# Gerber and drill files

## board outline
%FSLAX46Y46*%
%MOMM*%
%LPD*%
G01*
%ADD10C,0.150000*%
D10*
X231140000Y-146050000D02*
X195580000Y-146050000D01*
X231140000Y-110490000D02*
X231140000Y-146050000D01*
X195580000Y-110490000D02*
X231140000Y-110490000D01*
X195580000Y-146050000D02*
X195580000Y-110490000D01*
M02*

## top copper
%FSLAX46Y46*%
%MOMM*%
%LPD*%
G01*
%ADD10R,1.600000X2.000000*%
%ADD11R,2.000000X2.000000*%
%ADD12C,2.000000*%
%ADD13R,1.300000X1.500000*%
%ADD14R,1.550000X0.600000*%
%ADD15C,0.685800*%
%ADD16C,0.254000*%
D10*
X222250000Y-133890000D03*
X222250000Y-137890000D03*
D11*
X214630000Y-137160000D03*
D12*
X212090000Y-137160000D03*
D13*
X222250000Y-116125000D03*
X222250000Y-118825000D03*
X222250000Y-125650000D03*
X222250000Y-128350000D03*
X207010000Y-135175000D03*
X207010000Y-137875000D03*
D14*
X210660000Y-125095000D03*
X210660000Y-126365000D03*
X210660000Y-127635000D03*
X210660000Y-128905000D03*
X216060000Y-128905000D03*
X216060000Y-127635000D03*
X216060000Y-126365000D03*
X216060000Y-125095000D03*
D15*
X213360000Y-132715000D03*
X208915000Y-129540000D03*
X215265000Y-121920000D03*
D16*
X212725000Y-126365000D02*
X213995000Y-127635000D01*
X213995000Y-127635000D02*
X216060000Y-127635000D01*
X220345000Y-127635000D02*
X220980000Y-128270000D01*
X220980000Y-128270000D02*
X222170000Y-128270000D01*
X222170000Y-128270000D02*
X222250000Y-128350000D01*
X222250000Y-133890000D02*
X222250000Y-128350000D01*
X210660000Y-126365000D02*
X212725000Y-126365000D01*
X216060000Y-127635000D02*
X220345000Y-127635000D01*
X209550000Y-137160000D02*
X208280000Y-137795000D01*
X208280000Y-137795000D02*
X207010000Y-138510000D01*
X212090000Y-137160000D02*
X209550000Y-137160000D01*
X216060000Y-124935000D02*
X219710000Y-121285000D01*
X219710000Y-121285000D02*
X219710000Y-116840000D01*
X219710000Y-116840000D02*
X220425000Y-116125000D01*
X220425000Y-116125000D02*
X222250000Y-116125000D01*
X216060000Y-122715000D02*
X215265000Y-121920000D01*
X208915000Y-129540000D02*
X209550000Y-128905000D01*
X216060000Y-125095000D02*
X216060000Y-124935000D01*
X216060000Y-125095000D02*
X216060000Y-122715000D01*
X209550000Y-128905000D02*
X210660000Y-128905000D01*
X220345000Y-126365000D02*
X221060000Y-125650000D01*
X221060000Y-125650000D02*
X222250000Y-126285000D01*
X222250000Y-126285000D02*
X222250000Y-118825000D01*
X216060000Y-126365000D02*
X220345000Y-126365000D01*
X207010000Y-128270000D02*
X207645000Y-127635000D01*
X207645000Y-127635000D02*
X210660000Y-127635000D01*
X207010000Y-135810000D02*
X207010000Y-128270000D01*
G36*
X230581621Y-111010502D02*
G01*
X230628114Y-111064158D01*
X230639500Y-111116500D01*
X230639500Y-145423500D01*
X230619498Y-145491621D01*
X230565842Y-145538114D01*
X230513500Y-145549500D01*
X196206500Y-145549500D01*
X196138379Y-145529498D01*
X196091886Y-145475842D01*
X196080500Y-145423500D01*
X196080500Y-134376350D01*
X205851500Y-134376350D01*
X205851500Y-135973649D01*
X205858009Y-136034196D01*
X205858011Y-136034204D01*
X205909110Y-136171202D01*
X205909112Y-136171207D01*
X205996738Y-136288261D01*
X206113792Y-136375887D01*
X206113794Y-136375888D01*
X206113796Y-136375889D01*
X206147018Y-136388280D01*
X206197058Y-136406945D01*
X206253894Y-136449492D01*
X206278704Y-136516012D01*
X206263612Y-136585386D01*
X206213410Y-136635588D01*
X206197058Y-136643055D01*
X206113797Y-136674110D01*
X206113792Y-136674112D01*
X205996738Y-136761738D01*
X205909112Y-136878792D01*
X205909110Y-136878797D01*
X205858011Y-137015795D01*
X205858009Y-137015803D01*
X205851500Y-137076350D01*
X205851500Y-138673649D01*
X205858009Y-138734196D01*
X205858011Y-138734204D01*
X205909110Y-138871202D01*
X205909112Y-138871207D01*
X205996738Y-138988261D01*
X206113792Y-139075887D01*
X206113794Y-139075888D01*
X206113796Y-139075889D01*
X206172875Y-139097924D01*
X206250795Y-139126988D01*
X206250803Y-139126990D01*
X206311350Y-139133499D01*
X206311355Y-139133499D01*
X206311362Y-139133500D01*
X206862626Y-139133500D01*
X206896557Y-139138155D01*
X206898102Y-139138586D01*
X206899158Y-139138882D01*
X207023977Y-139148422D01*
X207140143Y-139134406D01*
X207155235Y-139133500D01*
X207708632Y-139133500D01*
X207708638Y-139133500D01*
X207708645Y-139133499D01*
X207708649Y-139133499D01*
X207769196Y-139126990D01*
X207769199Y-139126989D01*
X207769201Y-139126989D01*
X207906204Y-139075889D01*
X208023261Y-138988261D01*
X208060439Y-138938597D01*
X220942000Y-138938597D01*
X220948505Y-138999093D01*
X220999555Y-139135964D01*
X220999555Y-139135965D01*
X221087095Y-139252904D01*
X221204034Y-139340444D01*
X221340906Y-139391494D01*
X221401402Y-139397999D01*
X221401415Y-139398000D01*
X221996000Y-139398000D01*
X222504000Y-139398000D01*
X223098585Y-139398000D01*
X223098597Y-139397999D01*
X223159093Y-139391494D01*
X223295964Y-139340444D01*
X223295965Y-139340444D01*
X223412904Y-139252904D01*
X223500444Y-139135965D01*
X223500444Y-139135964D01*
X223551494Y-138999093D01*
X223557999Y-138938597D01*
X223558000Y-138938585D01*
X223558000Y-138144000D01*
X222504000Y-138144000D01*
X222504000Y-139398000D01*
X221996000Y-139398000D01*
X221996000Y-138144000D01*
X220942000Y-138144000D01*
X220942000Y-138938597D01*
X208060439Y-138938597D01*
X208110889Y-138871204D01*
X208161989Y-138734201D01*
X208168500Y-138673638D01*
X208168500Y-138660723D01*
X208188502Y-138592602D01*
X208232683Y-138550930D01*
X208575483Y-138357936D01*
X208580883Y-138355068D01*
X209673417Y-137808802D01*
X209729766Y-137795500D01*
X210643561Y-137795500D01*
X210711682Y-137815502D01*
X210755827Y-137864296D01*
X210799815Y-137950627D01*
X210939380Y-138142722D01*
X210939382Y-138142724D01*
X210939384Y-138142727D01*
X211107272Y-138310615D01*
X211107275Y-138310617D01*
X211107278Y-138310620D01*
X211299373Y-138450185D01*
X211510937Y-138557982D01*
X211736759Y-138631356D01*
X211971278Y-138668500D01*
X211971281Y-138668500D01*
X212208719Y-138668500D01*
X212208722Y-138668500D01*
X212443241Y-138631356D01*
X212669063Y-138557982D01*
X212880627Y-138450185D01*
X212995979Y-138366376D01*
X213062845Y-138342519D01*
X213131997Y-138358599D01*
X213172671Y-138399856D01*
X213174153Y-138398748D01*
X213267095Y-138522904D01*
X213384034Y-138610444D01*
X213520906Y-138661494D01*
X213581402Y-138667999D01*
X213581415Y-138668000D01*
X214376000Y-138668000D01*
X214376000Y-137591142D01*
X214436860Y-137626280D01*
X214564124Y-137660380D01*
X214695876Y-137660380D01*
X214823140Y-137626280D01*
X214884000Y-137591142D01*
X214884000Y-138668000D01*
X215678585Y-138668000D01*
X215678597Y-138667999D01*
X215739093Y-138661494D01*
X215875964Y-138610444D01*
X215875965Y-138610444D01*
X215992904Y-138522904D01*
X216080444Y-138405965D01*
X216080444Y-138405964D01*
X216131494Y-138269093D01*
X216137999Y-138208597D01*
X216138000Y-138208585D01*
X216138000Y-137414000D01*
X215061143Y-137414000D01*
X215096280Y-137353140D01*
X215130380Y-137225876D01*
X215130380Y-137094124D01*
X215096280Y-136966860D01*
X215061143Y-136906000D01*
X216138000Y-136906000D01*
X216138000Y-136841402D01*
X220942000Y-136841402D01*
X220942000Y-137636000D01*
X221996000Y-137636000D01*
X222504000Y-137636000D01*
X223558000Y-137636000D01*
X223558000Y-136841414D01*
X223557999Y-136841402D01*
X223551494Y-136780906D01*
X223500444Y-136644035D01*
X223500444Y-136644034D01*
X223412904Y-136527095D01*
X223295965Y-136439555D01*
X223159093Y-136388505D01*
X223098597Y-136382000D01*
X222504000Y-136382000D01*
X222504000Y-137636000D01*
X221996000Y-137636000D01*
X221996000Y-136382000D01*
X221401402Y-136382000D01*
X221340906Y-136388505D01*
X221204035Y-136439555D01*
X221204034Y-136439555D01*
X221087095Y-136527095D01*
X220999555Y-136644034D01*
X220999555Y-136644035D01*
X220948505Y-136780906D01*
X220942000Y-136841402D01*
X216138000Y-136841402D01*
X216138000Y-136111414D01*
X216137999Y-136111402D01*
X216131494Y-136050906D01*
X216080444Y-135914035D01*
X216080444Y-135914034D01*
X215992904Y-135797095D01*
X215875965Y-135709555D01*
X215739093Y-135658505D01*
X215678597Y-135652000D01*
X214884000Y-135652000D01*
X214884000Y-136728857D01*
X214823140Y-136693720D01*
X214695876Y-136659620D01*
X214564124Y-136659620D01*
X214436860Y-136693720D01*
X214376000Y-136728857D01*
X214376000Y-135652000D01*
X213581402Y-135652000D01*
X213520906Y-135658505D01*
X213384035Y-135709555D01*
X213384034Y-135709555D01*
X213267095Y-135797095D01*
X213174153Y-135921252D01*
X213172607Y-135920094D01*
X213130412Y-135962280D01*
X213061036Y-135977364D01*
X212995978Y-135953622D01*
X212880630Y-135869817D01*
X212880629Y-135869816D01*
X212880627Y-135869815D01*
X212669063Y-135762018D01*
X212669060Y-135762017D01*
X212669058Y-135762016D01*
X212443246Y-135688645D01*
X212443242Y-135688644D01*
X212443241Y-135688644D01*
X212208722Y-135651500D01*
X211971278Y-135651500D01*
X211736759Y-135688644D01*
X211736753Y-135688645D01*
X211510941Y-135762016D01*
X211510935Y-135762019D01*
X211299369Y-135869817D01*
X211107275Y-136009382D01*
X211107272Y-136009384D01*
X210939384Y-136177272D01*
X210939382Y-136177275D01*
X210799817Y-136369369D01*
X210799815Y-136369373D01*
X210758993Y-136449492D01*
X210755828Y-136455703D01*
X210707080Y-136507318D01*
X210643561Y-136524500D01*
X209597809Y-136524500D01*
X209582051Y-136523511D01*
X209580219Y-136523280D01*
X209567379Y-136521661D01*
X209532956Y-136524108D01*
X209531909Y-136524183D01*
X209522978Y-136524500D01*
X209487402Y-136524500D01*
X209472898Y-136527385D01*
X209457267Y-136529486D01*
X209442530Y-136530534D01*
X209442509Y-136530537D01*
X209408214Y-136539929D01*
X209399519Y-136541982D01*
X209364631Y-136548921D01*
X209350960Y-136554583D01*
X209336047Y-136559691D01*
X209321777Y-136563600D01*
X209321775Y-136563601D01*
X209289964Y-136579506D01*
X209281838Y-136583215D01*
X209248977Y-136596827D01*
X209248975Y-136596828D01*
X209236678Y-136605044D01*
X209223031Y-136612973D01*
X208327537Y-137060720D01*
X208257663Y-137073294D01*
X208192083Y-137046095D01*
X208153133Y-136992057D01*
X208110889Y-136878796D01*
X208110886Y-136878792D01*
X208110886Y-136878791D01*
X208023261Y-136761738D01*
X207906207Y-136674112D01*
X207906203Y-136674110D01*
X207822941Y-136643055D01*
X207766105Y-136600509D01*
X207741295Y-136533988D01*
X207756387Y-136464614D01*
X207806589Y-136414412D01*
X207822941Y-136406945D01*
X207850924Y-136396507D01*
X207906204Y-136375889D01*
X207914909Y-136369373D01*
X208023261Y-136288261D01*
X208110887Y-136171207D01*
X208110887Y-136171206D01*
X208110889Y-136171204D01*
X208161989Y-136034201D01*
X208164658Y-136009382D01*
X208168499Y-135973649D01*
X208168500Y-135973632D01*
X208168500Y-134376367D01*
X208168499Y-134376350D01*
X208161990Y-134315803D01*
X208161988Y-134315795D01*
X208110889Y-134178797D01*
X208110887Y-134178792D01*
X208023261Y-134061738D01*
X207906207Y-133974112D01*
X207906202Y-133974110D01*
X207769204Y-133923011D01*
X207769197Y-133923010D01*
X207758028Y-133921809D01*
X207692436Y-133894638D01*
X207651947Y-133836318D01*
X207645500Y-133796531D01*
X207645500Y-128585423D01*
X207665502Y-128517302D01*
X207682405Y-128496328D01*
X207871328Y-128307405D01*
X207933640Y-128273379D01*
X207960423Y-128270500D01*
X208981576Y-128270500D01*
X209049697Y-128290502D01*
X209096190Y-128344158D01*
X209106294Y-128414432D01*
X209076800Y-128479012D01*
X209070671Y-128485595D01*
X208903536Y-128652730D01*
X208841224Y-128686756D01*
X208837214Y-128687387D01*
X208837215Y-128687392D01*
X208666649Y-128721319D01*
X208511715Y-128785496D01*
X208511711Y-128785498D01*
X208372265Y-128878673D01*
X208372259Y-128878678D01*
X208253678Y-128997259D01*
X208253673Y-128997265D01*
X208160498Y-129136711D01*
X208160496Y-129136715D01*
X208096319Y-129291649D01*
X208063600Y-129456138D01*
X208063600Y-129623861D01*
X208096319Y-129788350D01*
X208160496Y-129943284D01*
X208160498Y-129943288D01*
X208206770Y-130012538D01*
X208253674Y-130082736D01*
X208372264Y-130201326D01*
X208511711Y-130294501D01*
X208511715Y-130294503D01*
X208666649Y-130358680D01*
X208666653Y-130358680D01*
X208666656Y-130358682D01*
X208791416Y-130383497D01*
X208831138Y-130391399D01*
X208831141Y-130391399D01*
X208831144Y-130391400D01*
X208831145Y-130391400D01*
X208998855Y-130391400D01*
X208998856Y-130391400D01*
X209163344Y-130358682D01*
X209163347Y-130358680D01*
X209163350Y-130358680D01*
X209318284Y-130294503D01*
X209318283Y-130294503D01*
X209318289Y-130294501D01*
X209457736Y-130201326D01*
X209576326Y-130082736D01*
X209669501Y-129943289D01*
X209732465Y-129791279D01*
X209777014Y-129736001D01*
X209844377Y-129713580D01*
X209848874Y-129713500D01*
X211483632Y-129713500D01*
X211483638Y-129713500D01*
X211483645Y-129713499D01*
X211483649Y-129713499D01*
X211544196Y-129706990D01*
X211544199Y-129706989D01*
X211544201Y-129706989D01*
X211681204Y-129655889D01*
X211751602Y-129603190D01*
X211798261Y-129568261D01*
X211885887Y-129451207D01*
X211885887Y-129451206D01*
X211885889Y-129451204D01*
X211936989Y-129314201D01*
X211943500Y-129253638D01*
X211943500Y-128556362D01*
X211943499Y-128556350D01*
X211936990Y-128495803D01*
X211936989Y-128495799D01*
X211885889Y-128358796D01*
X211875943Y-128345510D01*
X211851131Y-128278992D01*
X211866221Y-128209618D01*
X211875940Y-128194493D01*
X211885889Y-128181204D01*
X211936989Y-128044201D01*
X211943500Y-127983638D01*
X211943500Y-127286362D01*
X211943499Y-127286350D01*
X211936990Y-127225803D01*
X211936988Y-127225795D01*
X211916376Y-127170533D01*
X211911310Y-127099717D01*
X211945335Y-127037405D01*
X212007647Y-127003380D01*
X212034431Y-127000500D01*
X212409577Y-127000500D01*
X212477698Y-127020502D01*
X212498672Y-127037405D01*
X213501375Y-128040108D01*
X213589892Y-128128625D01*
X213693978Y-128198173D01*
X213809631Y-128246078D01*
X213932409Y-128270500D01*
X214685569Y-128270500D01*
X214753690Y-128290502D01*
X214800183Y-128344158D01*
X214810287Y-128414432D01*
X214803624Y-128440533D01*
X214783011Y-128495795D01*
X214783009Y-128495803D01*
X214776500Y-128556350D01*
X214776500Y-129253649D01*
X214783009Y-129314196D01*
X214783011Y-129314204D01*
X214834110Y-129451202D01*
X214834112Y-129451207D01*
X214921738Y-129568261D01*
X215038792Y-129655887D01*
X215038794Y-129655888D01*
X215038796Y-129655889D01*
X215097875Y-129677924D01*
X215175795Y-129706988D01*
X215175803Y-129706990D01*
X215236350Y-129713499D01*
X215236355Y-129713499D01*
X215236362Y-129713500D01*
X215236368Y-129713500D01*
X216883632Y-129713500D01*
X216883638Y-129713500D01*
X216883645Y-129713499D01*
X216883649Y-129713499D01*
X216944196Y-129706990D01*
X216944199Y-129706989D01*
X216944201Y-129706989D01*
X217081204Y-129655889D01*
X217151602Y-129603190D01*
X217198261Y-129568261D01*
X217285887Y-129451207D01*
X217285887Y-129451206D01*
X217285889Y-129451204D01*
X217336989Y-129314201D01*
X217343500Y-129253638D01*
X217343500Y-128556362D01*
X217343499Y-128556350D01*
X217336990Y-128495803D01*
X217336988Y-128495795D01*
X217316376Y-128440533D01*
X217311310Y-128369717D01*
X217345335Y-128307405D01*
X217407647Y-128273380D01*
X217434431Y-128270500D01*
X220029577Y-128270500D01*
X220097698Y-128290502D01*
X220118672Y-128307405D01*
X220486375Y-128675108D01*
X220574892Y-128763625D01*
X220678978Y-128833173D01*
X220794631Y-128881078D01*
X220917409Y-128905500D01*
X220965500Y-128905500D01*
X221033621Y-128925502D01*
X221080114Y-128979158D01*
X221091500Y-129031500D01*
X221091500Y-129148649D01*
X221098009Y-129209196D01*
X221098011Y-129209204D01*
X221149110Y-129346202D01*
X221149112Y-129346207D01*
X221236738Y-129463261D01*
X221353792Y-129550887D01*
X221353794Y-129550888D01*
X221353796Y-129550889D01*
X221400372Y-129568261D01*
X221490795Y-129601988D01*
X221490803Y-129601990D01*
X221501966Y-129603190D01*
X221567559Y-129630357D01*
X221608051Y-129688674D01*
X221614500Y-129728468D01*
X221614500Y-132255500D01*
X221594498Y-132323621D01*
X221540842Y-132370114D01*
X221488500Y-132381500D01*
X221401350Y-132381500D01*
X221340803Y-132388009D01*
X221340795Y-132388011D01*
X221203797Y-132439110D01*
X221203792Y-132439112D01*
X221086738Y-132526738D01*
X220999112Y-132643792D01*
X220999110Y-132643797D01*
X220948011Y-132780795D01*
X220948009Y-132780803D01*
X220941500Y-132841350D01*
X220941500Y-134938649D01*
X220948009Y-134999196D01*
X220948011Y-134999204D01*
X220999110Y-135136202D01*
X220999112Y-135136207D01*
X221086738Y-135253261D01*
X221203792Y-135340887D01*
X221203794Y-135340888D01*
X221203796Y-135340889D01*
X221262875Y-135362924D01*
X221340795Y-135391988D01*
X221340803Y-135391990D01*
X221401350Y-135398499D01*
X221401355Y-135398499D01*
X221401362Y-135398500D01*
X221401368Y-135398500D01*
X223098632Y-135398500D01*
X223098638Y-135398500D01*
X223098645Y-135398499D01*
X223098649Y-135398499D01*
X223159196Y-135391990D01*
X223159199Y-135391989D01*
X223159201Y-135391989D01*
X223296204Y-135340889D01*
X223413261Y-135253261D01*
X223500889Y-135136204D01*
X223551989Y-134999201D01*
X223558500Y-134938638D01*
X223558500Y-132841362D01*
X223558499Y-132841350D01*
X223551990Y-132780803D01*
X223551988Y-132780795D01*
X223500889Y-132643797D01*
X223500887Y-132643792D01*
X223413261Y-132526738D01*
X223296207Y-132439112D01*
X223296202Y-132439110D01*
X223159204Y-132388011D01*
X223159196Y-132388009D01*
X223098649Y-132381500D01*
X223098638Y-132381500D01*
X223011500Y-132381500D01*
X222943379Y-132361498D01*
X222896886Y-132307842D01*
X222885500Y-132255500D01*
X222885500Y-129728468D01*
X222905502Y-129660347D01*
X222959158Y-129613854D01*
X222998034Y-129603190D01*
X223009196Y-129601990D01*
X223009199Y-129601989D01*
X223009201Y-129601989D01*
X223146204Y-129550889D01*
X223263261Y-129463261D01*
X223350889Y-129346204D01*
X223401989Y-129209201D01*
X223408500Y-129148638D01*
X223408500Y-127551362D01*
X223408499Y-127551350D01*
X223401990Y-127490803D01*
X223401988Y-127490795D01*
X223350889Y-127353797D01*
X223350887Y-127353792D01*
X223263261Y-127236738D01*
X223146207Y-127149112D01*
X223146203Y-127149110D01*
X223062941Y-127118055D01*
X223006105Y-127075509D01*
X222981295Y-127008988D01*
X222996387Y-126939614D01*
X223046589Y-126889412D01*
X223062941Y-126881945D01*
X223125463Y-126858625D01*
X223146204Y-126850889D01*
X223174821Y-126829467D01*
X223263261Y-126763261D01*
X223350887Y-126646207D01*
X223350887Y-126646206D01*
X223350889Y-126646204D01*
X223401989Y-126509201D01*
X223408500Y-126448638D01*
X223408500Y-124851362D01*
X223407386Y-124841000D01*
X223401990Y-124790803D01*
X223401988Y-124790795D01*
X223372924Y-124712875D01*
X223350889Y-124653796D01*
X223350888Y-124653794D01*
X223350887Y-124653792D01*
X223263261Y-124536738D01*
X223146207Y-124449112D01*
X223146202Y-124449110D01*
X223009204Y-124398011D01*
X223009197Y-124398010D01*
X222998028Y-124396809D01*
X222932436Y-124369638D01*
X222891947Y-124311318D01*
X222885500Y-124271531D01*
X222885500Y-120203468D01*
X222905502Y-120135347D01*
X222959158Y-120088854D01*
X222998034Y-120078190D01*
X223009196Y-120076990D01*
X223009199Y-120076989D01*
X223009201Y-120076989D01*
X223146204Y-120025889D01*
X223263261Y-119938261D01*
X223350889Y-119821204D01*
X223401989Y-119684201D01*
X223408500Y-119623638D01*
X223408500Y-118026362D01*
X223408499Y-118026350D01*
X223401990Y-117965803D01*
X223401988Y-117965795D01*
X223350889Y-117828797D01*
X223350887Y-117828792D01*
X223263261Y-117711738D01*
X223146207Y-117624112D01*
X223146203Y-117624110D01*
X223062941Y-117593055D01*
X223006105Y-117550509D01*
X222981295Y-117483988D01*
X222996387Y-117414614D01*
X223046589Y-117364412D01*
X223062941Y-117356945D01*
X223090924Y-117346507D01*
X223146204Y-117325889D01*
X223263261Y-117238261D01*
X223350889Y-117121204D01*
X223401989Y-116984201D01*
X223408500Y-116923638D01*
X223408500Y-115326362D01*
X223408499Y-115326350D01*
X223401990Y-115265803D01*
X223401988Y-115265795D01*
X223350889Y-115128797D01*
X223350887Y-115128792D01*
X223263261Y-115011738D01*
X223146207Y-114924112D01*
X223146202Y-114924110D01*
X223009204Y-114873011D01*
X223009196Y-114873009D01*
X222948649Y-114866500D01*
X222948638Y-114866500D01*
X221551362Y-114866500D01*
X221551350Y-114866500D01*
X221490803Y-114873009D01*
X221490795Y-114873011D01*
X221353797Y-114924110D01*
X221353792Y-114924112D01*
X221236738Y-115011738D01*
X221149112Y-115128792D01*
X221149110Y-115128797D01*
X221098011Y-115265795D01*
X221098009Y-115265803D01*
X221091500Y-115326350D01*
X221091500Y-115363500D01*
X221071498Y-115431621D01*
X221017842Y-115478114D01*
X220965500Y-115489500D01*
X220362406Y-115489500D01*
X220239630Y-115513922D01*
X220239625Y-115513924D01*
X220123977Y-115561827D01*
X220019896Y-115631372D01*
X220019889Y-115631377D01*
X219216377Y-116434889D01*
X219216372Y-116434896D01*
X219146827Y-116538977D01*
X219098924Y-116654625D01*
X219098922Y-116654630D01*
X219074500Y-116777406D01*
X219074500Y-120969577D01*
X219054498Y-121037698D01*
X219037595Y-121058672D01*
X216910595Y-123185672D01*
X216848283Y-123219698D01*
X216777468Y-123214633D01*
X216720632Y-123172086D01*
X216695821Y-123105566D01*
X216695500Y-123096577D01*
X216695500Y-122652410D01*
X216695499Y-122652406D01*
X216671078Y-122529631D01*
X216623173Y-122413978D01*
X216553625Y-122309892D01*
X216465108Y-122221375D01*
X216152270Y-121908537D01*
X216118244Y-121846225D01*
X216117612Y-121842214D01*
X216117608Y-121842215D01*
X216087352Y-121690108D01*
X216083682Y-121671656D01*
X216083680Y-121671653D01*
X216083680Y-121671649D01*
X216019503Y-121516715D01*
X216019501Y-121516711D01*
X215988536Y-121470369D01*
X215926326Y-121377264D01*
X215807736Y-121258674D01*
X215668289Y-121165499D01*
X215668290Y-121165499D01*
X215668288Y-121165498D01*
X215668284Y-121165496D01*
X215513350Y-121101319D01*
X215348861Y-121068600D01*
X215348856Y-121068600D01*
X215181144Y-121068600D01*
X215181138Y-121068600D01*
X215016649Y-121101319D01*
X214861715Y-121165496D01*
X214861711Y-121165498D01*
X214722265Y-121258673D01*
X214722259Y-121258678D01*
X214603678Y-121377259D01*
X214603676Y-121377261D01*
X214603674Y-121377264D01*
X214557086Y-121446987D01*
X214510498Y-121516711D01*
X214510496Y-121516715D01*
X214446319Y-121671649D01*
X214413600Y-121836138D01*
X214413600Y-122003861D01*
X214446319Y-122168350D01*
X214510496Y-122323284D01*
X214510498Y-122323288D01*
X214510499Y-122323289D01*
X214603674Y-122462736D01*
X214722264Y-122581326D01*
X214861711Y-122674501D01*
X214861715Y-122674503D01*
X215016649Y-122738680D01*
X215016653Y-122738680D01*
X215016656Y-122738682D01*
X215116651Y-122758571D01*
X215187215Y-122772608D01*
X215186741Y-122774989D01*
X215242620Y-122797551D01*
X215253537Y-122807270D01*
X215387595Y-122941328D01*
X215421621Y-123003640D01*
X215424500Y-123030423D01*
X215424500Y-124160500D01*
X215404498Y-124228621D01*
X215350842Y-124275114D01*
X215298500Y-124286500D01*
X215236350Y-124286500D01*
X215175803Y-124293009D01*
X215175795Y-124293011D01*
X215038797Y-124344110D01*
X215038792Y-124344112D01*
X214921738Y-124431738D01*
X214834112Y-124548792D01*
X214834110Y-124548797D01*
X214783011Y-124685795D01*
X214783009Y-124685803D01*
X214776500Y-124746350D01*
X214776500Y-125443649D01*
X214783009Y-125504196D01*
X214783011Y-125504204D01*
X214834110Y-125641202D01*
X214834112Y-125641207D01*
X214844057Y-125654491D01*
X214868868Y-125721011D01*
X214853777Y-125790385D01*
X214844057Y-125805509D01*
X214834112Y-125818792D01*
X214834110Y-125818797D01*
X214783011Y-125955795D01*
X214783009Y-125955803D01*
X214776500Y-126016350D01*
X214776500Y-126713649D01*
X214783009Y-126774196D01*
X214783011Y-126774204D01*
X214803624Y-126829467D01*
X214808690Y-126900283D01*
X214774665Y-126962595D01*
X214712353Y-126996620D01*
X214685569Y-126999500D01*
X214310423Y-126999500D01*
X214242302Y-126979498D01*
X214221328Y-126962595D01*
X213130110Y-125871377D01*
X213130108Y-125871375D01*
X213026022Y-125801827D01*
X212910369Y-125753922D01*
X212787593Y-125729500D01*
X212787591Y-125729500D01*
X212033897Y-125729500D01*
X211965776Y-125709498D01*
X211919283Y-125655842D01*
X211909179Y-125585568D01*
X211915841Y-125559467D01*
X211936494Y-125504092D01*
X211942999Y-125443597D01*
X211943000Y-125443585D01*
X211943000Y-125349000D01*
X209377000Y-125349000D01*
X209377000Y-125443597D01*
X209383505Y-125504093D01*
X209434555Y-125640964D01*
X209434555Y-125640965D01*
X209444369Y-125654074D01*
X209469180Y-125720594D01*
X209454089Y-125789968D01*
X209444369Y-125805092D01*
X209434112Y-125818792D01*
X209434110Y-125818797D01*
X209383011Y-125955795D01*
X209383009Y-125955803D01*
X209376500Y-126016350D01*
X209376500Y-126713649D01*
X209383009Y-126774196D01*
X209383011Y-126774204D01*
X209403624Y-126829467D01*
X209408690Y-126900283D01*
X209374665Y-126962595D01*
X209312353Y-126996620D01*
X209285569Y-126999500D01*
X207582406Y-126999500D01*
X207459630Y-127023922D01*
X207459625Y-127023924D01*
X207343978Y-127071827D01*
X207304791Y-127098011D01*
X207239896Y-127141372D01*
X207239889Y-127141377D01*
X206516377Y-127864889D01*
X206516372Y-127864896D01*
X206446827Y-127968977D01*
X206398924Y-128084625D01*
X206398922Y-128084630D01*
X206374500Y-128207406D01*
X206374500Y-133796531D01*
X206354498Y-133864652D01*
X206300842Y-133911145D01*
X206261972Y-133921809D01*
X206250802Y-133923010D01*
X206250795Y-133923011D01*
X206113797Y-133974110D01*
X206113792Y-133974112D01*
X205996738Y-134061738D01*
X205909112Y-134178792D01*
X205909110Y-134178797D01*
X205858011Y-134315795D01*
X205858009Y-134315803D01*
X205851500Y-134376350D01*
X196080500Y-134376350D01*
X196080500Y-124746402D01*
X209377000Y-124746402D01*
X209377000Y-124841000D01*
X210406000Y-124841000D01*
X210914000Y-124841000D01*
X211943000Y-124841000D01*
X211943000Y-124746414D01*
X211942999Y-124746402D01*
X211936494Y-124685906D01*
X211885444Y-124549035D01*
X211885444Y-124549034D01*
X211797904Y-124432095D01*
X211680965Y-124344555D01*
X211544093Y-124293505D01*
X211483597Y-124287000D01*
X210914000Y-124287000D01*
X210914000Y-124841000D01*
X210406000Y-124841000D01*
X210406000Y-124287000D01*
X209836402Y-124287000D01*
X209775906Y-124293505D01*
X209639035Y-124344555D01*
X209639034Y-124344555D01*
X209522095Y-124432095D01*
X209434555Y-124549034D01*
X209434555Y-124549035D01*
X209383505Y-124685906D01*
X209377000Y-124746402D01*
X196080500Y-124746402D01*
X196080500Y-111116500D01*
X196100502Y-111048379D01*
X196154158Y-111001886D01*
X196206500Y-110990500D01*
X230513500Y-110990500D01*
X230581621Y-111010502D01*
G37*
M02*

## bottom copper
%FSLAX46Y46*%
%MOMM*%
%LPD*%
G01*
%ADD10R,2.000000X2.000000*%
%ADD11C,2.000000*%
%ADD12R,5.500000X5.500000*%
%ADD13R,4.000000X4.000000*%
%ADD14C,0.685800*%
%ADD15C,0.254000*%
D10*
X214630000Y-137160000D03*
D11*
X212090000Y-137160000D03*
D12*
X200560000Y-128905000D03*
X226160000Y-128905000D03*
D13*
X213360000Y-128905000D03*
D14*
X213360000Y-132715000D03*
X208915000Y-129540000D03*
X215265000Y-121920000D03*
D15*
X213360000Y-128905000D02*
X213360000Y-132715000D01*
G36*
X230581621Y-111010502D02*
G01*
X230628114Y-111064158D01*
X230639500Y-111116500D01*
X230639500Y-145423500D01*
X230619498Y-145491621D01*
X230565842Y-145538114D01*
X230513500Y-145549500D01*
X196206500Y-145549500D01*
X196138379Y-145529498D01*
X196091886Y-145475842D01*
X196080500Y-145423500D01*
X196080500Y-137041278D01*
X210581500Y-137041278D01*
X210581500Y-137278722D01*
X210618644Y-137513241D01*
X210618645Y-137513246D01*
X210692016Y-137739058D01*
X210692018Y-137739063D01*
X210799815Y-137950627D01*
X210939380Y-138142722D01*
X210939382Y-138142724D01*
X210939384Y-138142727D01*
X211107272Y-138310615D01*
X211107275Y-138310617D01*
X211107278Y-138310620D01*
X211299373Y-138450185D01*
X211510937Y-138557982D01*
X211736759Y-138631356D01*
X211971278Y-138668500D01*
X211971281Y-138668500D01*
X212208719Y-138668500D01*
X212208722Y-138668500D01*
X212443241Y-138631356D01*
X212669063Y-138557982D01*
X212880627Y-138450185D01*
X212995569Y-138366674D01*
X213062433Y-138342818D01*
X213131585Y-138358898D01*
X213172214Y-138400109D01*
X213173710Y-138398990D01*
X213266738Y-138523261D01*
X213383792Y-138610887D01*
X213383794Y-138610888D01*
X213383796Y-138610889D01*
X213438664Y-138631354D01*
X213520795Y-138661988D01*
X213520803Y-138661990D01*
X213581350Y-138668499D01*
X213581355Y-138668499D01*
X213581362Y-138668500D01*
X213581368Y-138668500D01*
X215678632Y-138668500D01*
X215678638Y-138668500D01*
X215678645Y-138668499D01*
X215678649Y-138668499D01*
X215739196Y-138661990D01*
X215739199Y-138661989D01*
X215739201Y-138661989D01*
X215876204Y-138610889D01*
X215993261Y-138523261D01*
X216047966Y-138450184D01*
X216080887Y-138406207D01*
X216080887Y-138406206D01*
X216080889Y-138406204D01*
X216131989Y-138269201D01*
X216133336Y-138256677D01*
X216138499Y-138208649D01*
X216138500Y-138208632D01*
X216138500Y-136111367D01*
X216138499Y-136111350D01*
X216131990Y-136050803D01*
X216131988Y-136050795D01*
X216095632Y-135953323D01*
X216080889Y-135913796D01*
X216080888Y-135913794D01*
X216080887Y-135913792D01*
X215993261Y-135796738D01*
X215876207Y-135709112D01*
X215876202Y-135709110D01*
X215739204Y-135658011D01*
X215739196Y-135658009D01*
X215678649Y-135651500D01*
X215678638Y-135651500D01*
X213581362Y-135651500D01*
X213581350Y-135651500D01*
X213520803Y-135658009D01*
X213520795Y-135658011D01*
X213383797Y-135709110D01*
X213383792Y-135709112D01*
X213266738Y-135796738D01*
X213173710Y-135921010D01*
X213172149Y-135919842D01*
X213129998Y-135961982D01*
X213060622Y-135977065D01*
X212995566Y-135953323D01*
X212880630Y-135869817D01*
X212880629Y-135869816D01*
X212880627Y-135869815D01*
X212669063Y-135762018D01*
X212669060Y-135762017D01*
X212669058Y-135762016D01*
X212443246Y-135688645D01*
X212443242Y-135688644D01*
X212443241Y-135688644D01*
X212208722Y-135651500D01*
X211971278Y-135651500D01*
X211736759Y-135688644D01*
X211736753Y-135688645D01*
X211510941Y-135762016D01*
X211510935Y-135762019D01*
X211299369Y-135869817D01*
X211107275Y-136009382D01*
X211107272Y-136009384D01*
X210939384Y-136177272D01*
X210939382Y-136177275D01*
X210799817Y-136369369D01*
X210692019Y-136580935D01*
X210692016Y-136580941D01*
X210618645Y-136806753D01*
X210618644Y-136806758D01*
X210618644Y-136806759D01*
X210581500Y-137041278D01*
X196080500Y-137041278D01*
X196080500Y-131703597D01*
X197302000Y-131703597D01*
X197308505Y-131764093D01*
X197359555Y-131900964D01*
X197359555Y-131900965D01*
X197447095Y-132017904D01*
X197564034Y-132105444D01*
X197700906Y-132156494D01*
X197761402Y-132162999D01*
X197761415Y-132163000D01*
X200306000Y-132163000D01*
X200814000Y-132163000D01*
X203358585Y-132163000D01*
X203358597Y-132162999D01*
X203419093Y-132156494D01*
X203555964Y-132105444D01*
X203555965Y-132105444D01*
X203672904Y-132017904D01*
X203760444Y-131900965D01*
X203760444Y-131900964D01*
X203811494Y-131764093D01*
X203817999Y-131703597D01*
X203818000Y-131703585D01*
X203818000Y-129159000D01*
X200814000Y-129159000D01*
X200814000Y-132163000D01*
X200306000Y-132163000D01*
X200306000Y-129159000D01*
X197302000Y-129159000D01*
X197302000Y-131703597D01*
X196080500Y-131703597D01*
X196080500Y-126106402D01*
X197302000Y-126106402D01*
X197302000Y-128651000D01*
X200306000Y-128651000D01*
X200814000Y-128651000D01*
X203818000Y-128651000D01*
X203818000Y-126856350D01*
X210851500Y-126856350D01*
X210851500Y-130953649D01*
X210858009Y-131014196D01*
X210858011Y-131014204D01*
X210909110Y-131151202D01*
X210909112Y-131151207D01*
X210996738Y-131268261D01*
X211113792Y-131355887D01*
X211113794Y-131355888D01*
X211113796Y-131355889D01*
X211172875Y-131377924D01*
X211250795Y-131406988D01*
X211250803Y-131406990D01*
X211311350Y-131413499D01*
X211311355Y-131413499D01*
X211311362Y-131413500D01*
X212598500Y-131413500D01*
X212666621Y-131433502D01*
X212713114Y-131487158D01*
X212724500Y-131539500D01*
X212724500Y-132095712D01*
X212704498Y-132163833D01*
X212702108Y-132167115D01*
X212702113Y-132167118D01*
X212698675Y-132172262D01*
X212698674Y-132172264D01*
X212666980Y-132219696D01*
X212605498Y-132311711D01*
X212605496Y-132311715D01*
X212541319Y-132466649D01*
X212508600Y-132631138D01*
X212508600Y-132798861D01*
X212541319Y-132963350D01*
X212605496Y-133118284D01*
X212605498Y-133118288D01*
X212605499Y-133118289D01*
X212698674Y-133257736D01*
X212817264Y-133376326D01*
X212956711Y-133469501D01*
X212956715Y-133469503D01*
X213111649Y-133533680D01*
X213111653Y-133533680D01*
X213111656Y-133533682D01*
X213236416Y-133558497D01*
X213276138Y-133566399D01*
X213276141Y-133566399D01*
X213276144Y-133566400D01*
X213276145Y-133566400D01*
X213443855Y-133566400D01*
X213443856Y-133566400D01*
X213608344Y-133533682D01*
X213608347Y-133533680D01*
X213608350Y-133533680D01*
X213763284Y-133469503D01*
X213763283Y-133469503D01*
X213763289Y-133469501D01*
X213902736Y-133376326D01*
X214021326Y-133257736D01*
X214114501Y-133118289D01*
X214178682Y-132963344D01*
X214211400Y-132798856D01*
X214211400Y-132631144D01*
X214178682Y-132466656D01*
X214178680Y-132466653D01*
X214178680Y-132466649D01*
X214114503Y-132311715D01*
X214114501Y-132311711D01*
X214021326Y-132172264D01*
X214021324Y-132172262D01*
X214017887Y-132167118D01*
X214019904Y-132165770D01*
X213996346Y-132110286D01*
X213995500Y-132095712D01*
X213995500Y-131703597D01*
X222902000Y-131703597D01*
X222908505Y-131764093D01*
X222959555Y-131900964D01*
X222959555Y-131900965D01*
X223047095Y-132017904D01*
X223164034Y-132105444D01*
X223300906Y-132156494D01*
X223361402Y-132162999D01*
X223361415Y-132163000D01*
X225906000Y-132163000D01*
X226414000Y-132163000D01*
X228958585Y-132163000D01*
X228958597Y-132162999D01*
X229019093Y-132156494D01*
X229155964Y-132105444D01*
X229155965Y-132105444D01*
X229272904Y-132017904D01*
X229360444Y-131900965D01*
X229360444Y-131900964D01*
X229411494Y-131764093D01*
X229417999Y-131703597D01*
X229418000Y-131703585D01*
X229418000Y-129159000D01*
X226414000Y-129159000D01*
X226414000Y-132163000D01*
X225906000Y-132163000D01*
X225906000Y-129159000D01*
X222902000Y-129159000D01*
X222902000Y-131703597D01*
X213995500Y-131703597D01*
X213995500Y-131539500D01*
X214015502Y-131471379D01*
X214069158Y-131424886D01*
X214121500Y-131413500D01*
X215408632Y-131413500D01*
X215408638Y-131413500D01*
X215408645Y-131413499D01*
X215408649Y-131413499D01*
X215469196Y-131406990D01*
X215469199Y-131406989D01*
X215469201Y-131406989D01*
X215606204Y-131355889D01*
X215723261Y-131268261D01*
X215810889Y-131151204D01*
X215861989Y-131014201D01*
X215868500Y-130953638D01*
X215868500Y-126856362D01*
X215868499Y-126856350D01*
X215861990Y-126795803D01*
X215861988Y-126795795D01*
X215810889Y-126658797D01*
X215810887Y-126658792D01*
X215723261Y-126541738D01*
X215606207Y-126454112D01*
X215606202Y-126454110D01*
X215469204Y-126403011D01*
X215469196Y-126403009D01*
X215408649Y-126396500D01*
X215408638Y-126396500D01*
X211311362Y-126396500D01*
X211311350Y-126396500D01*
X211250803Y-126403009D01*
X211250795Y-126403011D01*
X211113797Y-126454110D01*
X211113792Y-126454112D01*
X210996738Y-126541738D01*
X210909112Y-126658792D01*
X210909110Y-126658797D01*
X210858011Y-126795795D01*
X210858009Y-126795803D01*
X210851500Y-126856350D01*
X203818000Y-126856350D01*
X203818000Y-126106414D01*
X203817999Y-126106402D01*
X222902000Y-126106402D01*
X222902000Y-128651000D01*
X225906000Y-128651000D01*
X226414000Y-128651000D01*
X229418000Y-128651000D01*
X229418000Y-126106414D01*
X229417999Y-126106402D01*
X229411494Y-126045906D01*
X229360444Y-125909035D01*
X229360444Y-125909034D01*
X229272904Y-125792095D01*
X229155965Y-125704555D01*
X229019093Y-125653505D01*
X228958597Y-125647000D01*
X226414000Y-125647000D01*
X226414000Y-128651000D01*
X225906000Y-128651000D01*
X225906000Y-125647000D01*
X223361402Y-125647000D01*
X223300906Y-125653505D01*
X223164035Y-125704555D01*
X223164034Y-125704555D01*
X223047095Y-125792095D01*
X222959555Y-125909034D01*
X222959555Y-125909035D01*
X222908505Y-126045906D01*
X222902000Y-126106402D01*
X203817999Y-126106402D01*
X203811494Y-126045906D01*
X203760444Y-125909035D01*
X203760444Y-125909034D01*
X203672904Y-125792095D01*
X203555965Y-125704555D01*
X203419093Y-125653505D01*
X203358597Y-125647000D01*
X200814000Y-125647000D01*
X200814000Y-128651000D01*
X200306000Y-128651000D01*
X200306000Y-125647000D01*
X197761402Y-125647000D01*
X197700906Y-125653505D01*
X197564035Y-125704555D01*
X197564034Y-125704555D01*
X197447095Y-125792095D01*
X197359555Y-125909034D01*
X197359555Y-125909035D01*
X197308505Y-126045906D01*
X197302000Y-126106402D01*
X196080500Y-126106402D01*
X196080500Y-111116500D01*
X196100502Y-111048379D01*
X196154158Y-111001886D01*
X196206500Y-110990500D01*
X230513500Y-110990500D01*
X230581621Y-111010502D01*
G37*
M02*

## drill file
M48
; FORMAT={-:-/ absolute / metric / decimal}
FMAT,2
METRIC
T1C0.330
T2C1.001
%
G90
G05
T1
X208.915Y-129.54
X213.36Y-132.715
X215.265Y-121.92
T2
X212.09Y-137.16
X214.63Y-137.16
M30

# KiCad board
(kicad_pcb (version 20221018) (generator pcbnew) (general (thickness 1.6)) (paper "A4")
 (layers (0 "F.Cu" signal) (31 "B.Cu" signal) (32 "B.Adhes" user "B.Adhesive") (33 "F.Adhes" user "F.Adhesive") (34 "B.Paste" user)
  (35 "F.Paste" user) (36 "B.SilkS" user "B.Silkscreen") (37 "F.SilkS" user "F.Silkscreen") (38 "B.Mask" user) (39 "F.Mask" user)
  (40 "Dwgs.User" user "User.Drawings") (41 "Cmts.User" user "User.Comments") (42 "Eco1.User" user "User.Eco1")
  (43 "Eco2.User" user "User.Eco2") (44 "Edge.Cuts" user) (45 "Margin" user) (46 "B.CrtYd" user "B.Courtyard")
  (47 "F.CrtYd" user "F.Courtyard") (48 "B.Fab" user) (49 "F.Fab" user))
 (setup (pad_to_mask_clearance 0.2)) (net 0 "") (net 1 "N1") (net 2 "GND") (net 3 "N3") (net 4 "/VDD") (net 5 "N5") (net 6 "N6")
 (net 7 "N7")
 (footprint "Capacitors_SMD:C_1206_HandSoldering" (layer "F.Cu") (at 222.25 135.89 -90)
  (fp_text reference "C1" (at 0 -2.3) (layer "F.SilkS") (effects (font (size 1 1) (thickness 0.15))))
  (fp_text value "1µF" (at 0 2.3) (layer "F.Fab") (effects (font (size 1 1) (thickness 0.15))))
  (pad "1" smd rect (at -2 0 270) (size 2 1.6) (layers "F.Cu" "F.Paste" "F.Mask") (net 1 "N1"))
  (pad "2" smd rect (at 2 0 270) (size 2 1.6) (layers "F.Cu" "F.Paste" "F.Mask") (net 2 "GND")))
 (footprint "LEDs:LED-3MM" (layer "F.Cu") (at 214.63 137.16 180)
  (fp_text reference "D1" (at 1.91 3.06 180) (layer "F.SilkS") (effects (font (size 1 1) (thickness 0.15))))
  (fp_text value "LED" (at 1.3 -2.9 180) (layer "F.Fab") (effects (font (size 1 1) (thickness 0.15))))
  (pad "1" thru_hole rect (at 0 0 270) (size 2 2) (drill 1.00076) (layers "*.Cu" "*.Mask") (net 2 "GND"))
  (pad "2" thru_hole circle (at 2.54 0 180) (size 2 2) (drill 1.00076) (layers "*.Cu" "*.Mask") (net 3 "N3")))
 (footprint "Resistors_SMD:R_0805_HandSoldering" (layer "F.Cu") (at 222.25 117.475 -90)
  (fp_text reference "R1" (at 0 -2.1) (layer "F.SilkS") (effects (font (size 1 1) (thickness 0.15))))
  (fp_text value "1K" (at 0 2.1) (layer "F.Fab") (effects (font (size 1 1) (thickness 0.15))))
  (pad "1" smd rect (at -1.35 0 270) (size 1.5 1.3) (layers "F.Cu" "F.Paste" "F.Mask") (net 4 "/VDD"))
  (pad "2" smd rect (at 1.35 0 270) (size 1.5 1.3) (layers "F.Cu" "F.Paste" "F.Mask") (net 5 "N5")))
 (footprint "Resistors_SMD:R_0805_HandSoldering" (layer "F.Cu") (at 222.25 127 -90)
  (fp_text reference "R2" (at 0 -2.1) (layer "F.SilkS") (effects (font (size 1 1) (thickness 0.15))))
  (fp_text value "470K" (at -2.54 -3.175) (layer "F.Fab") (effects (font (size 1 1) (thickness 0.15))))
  (pad "1" smd rect (at -1.35 0 270) (size 1.5 1.3) (layers "F.Cu" "F.Paste" "F.Mask") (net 5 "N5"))
  (pad "2" smd rect (at 1.35 0 270) (size 1.5 1.3) (layers "F.Cu" "F.Paste" "F.Mask") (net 1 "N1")))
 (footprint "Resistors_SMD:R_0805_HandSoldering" (layer "F.Cu") (at 207.01 136.525 -90)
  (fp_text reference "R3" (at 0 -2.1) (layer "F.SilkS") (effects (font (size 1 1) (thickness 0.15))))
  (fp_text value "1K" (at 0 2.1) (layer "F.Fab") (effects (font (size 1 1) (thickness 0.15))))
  (pad "1" smd rect (at -1.35 0 270) (size 1.5 1.3) (layers "F.Cu" "F.Paste" "F.Mask") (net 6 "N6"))
  (pad "2" smd rect (at 1.35 0 270) (size 1.5 1.3) (layers "F.Cu" "F.Paste" "F.Mask") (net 3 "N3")))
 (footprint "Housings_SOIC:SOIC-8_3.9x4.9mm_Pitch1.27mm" (layer "F.Cu") (at 213.36 127)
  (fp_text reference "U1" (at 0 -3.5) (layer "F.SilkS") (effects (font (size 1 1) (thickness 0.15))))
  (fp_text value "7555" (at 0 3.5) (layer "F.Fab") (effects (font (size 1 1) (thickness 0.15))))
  (pad "1" smd rect (at -2.7 -1.905) (size 1.55 0.6) (layers "F.Cu" "F.Paste" "F.Mask") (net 2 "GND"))
  (pad "2" smd rect (at -2.7 -0.635) (size 1.55 0.6) (layers "F.Cu" "F.Paste" "F.Mask") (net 1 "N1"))
  (pad "3" smd rect (at -2.7 0.635) (size 1.55 0.6) (layers "F.Cu" "F.Paste" "F.Mask") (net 6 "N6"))
  (pad "4" smd rect (at -2.7 1.905) (size 1.55 0.6) (layers "F.Cu" "F.Paste" "F.Mask") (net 4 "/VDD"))
  (pad "5" smd rect (at 2.7 1.905) (size 1.55 0.6) (layers "F.Cu" "F.Paste" "F.Mask") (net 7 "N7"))
  (pad "6" smd rect (at 2.7 0.635) (size 1.55 0.6) (layers "F.Cu" "F.Paste" "F.Mask") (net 1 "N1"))
  (pad "7" smd rect (at 2.7 -0.635) (size 1.55 0.6) (layers "F.Cu" "F.Paste" "F.Mask") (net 5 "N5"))
  (pad "8" smd rect (at 2.7 -1.905) (size 1.55 0.6) (layers "F.Cu" "F.Paste" "F.Mask") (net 4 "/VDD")))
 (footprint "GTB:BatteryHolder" (layer "B.Cu") (at 213.36 128.905)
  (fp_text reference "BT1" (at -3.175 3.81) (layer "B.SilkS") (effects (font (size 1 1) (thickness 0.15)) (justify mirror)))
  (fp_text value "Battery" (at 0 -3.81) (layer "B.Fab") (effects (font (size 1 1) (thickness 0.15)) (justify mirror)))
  (pad "1" smd rect (at -12.8 0) (size 5.5 5.5) (layers "B.Cu" "B.Paste" "B.Mask") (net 4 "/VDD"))
  (pad "1" smd rect (at 12.8 0) (size 5.5 5.5) (layers "B.Cu" "B.Paste" "B.Mask") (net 4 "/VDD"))
  (pad "2" smd rect (at 0 0) (size 4 4) (layers "B.Cu" "B.Paste" "B.Mask") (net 2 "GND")))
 (gr_line (start 231.14 146.05) (end 195.58 146.05) (stroke (width 0.15) (type solid)) (layer "Edge.Cuts"))
 (gr_line (start 231.14 110.49) (end 231.14 146.05) (stroke (width 0.15) (type solid)) (layer "Edge.Cuts"))
 (gr_line (start 195.58 110.49) (end 231.14 110.49) (stroke (width 0.15) (type solid)) (layer "Edge.Cuts"))
 (gr_line (start 195.58 146.05) (end 195.58 110.49) (stroke (width 0.15) (type solid)) (layer "Edge.Cuts"))
 (segment (start 212.725 126.365) (end 213.995 127.635) (width 0.254) (layer "F.Cu") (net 1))
 (segment (start 213.995 127.635) (end 216.06 127.635) (width 0.254) (layer "F.Cu") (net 1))
 (segment (start 220.345 127.635) (end 220.98 128.27) (width 0.254) (layer "F.Cu") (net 1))
 (segment (start 220.98 128.27) (end 222.17 128.27) (width 0.254) (layer "F.Cu") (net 1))
 (segment (start 222.17 128.27) (end 222.25 128.35) (width 0.254) (layer "F.Cu") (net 1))
 (segment (start 222.25 133.89) (end 222.25 128.35) (width 0.254) (layer "F.Cu") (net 1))
 (segment (start 210.66 126.365) (end 212.725 126.365) (width 0.254) (layer "F.Cu") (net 1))
 (segment (start 216.06 127.635) (end 220.345 127.635) (width 0.254) (layer "F.Cu") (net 1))
 (via (at 213.36 132.715) (size 0.6858) (drill 0.3302) (layers "F.Cu" "B.Cu") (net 2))
 (segment (start 213.36 128.905) (end 213.36 132.715) (width 0.254) (layer "B.Cu") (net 2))
 (segment (start 209.55 137.16) (end 208.28 137.795) (width 0.254) (layer "F.Cu") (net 3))
 (segment (start 208.28 137.795) (end 207.01 138.51) (width 0.254) (layer "F.Cu") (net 3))
 (segment (start 212.09 137.16) (end 209.55 137.16) (width 0.254) (layer "F.Cu") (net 3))
 (segment (start 216.06 124.935) (end 219.71 121.285) (width 0.254) (layer "F.Cu") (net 4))
 (segment (start 219.71 121.285) (end 219.71 116.84) (width 0.254) (layer "F.Cu") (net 4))
 (segment (start 219.71 116.84) (end 220.425 116.125) (width 0.254) (layer "F.Cu") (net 4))
 (segment (start 220.425 116.125) (end 222.25 116.125) (width 0.254) (layer "F.Cu") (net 4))
 (segment (start 216.06 122.715) (end 215.265 121.92) (width 0.254) (layer "F.Cu") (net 4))
 (segment (start 208.915 129.54) (end 209.55 128.905) (width 0.254) (layer "F.Cu") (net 4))
 (segment (start 216.06 125.095) (end 216.06 124.935) (width 0.254) (layer "F.Cu") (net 4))
 (segment (start 216.06 125.095) (end 216.06 122.715) (width 0.254) (layer "F.Cu") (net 4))
 (segment (start 209.55 128.905) (end 210.66 128.905) (width 0.254) (layer "F.Cu") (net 4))
 (via (at 208.915 129.54) (size 0.6858) (drill 0.3302) (layers "F.Cu" "B.Cu") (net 4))
 (via (at 215.265 121.92) (size 0.6858) (drill 0.3302) (layers "F.Cu" "B.Cu") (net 4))
 (segment (start 220.345 126.365) (end 221.06 125.65) (width 0.254) (layer "F.Cu") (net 5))
 (segment (start 221.06 125.65) (end 222.25 126.285) (width 0.254) (layer "F.Cu") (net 5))
 (segment (start 222.25 126.285) (end 222.25 118.825) (width 0.254) (layer "F.Cu") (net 5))
 (segment (start 216.06 126.365) (end 220.345 126.365) (width 0.254) (layer "F.Cu") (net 5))
 (segment (start 207.01 128.27) (end 207.645 127.635) (width 0.254) (layer "F.Cu") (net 6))
 (segment (start 207.645 127.635) (end 210.66 127.635) (width 0.254) (layer "F.Cu") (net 6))
 (segment (start 207.01 135.81) (end 207.01 128.27) (width 0.254) (layer "F.Cu") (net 6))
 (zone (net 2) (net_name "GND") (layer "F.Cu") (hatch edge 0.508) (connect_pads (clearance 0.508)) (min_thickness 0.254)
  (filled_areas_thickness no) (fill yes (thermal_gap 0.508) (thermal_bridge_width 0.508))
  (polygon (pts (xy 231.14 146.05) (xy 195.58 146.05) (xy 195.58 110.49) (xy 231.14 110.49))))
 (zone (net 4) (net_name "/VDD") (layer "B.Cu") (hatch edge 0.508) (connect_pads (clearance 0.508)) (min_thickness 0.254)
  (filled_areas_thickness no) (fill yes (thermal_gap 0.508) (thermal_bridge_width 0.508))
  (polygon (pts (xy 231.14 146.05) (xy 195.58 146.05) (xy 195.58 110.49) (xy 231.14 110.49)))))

